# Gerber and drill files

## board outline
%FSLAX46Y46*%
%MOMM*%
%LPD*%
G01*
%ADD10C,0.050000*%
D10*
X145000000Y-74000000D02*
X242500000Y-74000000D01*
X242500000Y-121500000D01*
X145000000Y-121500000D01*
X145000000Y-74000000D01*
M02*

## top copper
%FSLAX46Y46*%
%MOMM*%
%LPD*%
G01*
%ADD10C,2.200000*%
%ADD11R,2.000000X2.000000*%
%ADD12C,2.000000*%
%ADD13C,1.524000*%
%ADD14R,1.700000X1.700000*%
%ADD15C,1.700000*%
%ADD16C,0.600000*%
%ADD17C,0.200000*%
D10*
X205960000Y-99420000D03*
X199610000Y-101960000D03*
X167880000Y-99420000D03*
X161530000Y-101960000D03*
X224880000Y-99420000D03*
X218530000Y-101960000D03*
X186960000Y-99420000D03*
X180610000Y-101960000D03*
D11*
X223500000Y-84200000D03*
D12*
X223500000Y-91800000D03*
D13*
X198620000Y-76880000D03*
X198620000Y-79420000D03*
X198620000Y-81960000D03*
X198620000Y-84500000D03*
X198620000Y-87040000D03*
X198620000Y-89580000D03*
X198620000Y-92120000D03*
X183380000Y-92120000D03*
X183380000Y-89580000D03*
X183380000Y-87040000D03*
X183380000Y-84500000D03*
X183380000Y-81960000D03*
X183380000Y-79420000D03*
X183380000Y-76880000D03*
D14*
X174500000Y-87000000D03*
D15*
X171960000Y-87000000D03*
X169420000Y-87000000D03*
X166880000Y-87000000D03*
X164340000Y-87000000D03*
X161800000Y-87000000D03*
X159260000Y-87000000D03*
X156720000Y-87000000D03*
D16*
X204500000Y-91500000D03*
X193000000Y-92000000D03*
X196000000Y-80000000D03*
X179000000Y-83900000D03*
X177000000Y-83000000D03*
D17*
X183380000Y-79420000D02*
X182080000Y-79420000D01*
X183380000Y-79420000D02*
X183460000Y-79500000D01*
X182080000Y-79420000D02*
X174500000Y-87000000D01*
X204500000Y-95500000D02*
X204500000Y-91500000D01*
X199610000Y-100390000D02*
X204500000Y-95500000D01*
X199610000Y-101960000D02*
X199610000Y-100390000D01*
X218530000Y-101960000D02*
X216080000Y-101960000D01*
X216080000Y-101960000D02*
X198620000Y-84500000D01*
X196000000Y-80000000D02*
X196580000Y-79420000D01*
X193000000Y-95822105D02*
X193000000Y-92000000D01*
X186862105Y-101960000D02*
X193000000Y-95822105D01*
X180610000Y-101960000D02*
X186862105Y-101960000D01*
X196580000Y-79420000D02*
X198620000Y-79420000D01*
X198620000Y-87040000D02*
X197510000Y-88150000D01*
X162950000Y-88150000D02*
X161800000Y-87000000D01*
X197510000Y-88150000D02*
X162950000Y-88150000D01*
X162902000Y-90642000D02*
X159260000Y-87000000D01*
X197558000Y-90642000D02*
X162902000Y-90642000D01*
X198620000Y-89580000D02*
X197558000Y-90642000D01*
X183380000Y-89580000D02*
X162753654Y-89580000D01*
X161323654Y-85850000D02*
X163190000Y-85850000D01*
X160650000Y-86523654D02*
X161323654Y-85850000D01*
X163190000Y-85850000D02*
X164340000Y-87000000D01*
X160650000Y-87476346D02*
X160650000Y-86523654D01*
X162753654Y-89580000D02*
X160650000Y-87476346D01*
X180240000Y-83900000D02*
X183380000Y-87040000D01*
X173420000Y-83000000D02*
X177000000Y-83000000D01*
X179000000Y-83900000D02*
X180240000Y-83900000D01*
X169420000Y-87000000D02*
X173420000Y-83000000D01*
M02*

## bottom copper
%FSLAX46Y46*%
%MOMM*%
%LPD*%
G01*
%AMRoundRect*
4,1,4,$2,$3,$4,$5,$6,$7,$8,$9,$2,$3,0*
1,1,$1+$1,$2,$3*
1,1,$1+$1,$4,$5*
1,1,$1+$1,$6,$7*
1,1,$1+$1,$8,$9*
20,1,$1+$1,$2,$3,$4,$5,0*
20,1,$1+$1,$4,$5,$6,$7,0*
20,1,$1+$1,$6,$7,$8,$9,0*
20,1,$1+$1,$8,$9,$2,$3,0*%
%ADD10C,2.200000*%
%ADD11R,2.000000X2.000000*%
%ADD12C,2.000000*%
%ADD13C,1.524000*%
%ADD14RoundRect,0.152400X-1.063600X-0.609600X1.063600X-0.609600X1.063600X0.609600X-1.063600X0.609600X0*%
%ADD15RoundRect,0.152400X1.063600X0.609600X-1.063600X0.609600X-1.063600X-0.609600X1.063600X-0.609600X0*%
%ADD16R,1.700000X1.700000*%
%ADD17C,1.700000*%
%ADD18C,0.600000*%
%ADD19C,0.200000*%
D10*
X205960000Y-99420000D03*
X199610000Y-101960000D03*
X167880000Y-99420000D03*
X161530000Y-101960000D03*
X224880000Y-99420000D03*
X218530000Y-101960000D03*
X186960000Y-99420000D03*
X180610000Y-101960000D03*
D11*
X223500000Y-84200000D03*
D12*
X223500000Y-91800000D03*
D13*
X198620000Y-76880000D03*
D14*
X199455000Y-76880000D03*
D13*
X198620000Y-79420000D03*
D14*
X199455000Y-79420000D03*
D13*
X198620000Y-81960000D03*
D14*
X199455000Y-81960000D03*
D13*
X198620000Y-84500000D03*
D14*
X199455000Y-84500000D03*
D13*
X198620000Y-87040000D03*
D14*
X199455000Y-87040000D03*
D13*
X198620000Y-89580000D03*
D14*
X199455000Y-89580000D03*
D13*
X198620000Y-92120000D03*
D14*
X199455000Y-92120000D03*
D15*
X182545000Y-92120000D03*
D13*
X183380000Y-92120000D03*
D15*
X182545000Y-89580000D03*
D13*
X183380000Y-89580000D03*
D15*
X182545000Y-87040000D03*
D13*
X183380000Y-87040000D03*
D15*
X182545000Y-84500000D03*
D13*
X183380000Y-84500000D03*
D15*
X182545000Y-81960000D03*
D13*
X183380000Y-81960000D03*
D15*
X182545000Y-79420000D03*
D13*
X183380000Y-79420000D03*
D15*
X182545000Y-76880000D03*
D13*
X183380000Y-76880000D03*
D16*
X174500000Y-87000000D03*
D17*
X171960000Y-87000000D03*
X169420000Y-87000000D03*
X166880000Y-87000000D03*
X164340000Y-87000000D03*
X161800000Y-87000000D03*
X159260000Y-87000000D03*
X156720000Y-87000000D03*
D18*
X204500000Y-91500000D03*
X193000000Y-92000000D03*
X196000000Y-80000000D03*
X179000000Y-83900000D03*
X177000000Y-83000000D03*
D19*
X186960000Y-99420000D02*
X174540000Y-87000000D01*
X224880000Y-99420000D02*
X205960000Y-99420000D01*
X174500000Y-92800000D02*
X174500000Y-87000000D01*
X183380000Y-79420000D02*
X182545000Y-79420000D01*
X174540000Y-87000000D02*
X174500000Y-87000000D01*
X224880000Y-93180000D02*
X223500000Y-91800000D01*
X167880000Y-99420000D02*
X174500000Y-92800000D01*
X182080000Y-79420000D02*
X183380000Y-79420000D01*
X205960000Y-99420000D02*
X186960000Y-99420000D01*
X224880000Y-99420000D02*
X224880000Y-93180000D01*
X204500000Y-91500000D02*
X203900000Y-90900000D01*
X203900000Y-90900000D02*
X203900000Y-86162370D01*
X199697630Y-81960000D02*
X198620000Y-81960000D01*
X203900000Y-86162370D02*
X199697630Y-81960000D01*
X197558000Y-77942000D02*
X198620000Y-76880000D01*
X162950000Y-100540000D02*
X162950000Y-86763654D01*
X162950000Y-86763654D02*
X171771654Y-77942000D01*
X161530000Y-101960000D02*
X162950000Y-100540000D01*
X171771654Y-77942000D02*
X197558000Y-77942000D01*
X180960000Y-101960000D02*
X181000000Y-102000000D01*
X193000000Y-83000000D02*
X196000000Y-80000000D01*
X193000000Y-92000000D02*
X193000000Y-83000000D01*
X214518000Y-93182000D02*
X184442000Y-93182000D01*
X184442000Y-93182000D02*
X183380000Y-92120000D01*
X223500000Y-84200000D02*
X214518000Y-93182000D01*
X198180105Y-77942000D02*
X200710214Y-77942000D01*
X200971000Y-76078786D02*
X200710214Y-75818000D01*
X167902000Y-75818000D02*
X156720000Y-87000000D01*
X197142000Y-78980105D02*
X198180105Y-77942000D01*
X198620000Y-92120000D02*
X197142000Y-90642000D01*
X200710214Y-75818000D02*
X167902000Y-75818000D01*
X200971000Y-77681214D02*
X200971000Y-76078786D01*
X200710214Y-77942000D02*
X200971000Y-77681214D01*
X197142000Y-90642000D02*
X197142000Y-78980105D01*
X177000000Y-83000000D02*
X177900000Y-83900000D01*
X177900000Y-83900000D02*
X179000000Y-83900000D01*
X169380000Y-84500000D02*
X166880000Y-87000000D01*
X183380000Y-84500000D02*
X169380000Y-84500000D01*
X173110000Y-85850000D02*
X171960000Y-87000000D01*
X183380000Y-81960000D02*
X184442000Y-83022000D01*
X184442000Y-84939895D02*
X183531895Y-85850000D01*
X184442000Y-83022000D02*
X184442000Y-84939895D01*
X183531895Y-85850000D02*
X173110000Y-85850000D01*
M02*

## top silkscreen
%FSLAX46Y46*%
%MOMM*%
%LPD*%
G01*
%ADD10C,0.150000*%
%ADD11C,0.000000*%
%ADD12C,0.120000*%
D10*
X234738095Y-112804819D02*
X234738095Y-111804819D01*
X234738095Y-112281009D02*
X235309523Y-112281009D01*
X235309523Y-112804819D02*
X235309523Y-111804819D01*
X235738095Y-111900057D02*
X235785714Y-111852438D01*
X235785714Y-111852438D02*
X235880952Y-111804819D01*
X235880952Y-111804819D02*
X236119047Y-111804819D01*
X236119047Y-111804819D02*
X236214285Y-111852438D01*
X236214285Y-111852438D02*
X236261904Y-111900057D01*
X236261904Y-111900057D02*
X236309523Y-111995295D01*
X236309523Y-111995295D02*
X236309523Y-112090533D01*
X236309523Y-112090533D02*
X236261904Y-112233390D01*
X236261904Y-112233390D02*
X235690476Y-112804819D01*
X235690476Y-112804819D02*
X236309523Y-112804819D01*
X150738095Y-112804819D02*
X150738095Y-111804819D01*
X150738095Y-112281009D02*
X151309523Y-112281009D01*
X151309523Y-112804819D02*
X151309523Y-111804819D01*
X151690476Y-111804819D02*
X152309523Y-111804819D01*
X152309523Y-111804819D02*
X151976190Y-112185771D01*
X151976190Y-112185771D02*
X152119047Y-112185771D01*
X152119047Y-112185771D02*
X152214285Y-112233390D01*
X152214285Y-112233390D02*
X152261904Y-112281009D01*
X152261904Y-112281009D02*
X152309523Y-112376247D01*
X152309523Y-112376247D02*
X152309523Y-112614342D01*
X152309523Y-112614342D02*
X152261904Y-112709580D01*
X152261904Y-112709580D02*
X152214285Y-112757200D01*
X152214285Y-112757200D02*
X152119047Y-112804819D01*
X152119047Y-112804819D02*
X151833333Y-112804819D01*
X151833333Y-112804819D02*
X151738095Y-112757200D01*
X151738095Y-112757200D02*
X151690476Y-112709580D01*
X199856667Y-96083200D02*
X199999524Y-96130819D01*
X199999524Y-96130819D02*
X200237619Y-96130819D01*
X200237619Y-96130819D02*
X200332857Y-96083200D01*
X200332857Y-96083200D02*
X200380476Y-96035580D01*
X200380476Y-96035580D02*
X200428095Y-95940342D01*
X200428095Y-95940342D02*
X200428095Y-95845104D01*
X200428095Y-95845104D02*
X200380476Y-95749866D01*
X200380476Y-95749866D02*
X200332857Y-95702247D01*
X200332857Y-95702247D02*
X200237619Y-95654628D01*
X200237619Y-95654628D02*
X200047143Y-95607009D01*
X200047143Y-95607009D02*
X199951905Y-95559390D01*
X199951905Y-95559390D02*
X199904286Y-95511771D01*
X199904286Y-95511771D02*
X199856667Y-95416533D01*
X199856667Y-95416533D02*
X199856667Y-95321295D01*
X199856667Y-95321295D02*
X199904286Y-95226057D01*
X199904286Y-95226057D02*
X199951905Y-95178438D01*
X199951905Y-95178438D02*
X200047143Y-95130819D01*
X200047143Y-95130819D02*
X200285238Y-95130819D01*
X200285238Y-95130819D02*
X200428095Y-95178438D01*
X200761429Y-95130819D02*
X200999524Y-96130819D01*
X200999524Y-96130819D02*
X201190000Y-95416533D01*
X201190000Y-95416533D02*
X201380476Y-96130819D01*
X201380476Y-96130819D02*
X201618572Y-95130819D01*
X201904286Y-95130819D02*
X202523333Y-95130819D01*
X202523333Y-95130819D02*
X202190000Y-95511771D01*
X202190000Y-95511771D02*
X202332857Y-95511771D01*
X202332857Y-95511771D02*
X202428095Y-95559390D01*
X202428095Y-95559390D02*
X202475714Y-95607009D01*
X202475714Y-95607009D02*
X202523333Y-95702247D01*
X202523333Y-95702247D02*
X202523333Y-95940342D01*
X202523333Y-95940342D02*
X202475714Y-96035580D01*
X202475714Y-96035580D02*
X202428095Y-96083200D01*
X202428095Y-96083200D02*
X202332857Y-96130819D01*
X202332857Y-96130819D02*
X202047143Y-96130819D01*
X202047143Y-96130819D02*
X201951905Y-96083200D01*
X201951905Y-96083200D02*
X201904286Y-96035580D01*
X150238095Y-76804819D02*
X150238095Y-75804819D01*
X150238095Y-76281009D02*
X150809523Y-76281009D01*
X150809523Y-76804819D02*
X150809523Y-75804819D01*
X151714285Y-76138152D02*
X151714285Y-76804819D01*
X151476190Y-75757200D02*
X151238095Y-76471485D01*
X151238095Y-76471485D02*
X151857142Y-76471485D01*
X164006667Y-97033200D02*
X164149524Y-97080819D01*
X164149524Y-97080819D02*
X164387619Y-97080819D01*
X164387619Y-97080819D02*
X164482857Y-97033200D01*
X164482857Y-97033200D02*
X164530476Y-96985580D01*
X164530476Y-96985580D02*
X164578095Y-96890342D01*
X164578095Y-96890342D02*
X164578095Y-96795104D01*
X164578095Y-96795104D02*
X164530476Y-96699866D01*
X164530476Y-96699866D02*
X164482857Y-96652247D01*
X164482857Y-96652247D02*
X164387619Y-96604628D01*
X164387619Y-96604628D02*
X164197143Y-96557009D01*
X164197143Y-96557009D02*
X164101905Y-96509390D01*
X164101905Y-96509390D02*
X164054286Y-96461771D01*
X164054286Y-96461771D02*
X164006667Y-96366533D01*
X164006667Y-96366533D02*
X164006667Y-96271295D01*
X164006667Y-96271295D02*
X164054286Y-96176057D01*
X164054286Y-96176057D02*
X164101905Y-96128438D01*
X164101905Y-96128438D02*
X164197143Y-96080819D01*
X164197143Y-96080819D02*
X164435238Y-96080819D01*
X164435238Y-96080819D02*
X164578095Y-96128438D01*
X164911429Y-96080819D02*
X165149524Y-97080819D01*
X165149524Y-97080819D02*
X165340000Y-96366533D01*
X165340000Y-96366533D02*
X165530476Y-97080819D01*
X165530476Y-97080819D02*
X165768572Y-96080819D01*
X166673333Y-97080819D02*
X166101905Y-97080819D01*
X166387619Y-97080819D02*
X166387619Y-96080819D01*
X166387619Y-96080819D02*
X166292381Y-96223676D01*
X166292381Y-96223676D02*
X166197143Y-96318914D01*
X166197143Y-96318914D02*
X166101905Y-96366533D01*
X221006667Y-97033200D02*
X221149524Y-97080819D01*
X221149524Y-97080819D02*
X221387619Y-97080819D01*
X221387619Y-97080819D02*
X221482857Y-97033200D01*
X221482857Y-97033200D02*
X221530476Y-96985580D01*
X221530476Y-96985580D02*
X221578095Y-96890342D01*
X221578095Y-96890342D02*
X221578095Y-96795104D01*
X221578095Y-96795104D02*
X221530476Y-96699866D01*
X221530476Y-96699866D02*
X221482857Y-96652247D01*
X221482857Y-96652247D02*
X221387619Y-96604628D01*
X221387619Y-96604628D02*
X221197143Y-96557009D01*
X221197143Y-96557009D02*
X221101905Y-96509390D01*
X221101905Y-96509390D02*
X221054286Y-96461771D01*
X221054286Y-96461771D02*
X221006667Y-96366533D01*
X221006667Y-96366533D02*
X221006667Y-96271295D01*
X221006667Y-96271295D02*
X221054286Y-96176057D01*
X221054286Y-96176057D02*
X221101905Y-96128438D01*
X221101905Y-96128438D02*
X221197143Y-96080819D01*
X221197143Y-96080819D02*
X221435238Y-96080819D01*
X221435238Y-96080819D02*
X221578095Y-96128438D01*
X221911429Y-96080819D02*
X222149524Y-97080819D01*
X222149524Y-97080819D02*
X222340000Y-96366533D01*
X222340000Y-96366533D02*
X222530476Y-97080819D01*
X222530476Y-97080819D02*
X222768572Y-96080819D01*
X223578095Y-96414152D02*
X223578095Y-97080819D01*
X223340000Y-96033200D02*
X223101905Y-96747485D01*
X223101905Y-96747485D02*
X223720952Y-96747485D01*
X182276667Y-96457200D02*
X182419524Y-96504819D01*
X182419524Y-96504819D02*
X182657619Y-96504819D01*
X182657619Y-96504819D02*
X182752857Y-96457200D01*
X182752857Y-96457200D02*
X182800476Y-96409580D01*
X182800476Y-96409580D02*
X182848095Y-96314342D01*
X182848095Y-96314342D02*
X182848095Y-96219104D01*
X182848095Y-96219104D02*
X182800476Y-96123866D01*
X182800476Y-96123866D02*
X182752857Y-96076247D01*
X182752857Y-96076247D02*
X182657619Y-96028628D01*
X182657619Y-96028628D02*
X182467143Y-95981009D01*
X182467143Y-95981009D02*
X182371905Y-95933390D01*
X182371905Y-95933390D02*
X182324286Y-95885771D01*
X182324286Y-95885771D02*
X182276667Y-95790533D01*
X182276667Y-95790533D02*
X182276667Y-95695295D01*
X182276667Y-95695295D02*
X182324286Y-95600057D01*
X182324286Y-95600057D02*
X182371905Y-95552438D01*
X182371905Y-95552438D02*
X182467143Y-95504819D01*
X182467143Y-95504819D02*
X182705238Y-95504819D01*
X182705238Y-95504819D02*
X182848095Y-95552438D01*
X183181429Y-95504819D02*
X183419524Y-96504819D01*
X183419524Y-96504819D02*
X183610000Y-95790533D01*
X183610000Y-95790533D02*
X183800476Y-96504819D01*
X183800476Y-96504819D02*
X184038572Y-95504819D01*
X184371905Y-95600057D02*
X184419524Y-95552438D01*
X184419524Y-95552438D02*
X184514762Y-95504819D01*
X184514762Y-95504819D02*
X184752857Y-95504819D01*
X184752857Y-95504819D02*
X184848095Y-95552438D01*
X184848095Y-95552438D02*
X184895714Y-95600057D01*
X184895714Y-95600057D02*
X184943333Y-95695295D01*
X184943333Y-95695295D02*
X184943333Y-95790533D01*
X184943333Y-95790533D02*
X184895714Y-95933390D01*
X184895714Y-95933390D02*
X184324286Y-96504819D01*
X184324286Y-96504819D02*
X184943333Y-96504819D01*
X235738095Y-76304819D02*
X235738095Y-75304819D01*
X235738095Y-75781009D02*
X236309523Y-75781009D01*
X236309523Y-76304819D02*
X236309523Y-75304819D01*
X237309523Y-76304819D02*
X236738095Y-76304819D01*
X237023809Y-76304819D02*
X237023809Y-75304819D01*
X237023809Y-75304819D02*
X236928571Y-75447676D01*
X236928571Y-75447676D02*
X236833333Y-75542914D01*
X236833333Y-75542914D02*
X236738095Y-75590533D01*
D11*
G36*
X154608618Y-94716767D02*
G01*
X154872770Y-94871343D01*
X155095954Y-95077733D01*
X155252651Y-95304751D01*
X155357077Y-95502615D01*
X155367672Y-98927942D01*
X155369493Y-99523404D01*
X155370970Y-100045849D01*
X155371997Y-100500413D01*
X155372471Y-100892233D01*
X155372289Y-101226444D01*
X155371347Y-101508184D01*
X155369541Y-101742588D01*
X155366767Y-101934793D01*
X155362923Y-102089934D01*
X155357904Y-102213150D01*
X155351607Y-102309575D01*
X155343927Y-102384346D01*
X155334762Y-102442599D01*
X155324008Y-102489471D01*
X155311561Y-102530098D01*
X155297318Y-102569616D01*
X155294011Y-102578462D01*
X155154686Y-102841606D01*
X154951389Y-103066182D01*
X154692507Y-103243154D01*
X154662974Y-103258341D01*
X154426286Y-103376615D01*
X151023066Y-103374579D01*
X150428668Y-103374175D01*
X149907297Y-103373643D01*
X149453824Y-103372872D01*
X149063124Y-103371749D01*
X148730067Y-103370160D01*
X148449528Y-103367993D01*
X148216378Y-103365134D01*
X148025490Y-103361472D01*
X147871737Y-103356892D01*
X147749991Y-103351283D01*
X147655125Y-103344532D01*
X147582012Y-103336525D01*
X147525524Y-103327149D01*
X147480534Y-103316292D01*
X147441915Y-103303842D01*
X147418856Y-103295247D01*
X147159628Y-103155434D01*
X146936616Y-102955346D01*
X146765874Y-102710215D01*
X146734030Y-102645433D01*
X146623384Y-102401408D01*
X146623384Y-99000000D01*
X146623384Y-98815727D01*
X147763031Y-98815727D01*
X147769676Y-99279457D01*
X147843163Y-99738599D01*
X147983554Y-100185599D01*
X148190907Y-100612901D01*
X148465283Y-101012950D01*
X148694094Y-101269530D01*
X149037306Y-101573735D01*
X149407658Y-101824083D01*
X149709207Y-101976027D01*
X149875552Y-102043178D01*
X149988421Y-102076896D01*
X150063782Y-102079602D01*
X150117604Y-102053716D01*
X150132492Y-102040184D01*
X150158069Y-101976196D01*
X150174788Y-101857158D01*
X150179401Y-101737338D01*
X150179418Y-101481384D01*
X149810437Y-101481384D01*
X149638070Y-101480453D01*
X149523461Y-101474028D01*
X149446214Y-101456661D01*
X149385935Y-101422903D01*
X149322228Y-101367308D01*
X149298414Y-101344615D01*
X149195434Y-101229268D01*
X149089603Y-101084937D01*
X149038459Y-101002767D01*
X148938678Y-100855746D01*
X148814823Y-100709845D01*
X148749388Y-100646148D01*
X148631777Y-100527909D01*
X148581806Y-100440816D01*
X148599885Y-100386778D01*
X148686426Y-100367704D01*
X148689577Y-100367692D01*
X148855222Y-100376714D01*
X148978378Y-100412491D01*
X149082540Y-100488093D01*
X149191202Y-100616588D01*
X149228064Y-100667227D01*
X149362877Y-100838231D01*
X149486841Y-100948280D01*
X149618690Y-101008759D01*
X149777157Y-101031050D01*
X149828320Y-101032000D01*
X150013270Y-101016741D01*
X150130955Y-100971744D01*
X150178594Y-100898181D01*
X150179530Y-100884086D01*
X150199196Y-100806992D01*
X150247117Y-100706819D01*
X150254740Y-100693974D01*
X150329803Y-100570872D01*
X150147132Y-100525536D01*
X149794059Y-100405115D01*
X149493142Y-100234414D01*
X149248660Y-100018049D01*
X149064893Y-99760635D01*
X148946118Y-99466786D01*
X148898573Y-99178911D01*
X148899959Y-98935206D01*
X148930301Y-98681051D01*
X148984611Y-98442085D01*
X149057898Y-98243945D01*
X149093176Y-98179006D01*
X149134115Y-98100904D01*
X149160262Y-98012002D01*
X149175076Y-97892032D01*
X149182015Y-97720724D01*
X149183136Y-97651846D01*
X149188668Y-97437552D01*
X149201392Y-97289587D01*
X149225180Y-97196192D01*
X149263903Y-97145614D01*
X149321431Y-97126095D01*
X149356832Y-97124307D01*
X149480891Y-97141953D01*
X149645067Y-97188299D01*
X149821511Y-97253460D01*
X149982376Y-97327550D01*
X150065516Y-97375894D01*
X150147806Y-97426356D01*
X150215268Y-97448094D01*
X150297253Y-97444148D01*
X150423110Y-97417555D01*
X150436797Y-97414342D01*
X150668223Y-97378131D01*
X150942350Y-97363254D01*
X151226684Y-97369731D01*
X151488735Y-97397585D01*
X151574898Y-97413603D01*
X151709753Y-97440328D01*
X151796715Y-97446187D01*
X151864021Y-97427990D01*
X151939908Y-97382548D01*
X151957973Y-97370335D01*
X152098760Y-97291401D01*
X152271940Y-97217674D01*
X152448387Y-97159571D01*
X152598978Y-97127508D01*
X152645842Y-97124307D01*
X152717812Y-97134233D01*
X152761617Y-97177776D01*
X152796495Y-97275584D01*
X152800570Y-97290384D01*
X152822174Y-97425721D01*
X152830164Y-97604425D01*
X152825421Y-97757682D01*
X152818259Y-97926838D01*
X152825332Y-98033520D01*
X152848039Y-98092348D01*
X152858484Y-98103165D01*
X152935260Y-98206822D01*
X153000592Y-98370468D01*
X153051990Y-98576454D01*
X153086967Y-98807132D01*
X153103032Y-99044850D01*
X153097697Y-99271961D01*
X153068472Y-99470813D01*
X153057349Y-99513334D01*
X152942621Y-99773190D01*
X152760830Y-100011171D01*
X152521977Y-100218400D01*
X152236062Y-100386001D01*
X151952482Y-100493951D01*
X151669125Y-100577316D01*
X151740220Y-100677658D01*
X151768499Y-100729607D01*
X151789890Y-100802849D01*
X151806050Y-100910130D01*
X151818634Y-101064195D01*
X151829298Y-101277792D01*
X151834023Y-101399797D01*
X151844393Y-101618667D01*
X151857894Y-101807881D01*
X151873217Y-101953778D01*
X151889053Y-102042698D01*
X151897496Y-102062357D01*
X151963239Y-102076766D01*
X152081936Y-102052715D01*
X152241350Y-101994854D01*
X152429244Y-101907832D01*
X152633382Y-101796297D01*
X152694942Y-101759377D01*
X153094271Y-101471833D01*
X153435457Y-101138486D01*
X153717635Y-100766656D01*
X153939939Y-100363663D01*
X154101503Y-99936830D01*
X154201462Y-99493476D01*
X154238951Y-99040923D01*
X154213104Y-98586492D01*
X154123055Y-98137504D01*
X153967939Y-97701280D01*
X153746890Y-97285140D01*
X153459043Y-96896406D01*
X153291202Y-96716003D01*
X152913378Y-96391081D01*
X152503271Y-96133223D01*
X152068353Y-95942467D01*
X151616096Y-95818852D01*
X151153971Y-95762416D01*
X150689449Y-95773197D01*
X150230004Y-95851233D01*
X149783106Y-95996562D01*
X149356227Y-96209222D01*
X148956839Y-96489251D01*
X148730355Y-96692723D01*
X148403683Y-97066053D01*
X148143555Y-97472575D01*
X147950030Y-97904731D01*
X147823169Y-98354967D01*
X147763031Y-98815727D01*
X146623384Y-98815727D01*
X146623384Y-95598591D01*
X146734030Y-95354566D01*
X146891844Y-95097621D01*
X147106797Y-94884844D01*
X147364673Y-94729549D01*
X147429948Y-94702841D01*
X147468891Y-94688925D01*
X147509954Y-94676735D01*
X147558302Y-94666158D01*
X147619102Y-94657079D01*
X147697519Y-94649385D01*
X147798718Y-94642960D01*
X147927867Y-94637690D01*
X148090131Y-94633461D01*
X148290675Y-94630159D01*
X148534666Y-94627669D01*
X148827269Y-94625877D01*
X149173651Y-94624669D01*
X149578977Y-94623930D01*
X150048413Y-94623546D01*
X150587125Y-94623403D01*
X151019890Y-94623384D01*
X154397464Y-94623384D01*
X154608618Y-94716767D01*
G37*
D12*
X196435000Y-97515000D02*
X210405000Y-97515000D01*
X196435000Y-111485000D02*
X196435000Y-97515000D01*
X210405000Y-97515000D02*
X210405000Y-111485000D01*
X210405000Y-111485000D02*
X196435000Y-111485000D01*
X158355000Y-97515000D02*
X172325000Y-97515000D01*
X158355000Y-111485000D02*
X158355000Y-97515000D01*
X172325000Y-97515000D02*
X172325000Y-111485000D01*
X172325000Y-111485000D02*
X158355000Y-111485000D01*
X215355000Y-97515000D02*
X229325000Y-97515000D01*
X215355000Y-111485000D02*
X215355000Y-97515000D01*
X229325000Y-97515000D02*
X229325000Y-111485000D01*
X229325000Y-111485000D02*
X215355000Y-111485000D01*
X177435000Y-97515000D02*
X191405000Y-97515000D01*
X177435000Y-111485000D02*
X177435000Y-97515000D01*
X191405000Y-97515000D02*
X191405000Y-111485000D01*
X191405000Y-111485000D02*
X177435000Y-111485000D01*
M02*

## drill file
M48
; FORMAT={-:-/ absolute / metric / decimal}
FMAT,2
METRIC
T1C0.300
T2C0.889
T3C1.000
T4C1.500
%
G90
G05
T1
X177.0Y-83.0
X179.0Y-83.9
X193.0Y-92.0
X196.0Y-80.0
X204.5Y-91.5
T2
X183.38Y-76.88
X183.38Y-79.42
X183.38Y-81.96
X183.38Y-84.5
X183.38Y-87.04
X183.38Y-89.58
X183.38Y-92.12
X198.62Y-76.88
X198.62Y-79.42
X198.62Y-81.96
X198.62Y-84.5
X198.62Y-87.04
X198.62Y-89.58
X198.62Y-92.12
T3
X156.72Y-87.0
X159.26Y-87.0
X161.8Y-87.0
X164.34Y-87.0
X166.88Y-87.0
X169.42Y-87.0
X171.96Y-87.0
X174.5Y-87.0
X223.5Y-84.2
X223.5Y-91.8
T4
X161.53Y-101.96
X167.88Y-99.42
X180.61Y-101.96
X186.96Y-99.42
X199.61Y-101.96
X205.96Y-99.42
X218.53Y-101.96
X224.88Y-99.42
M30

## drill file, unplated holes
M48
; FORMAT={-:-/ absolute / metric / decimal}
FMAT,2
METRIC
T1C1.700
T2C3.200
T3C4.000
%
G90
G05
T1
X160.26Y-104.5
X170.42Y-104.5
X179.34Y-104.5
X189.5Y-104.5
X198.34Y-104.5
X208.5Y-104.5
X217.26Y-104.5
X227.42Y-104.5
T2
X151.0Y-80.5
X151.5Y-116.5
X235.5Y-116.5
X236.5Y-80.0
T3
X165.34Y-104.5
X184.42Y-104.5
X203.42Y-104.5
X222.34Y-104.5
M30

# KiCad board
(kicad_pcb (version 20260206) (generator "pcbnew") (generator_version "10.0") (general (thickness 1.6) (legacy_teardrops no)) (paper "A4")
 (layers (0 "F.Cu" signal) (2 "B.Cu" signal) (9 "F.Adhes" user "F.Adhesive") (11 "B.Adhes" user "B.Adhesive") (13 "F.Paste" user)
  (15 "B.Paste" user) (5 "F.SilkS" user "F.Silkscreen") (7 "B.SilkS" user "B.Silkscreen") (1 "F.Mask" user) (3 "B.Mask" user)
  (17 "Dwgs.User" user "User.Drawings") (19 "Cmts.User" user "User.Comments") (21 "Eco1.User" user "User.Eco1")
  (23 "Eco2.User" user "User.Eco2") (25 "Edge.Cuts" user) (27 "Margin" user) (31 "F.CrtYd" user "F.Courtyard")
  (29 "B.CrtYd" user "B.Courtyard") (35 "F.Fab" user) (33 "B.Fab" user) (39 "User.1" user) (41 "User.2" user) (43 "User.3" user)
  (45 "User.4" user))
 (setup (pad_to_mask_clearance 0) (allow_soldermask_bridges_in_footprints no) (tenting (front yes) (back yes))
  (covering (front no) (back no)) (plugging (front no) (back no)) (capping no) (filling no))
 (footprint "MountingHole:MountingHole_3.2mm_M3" (layer "F.Cu") (at 235.5 116.5)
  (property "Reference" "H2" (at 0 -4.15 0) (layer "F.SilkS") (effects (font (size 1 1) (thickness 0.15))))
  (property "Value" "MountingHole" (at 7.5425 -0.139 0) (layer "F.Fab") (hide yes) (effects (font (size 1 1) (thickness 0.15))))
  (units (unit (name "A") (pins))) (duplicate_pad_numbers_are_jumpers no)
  (pad "" np_thru_hole circle (at 0 0) (size 3.2 3.2) (drill 3.2) (layers "*.Cu" "*.Mask")))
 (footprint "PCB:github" (layer "F.Cu") (at 151 99)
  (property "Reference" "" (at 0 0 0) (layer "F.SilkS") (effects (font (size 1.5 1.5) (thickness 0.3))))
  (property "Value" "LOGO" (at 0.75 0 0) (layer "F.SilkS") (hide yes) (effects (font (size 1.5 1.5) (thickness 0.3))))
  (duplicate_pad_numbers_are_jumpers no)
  (fp_poly
   (pts (xy 3.608618 -4.283233) (xy 3.87277 -4.128657) (xy 4.095954 -3.922267) (xy 4.252651 -3.695249) (xy 4.357077 -3.497385)
    (xy 4.367672 -0.072058) (xy 4.369493 0.523404) (xy 4.37097 1.045849) (xy 4.371997 1.500413) (xy 4.372471 1.892233)
    (xy 4.372289 2.226444) (xy 4.371347 2.508184) (xy 4.369541 2.742588) (xy 4.366767 2.934793) (xy 4.362923 3.089934) (xy 4.357904 3.21315)
    (xy 4.351607 3.309575) (xy 4.343927 3.384346) (xy 4.334762 3.442599) (xy 4.324008 3.489471) (xy 4.311561 3.530098)
    (xy 4.297318 3.569616) (xy 4.294011 3.578462) (xy 4.154686 3.841606) (xy 3.951389 4.066182) (xy 3.692507 4.243154)
    (xy 3.662974 4.258341) (xy 3.426286 4.376615) (xy 0.023066 4.374579) (xy -0.571332 4.374175) (xy -1.092703 4.373643)
    (xy -1.546176 4.372872) (xy -1.936876 4.371749) (xy -2.269933 4.37016) (xy -2.550472 4.367993) (xy -2.783622 4.365134)
    (xy -2.97451 4.361472) (xy -3.128263 4.356892) (xy -3.250009 4.351283) (xy -3.344875 4.344532) (xy -3.417988 4.336525)
    (xy -3.474476 4.327149) (xy -3.519466 4.316292) (xy -3.558085 4.303842) (xy -3.581144 4.295247) (xy -3.840372 4.155434)
    (xy -4.063384 3.955346) (xy -4.234126 3.710215) (xy -4.26597 3.645433) (xy -4.376616 3.401408) (xy -4.376616 0) (xy -4.376616 -0.184273)
    (xy -3.236969 -0.184273) (xy -3.230324 0.279457) (xy -3.156837 0.738599) (xy -3.016446 1.185599) (xy -2.809093 1.612901)
    (xy -2.534717 2.01295) (xy -2.305906 2.26953) (xy -1.962694 2.573735) (xy -1.592342 2.824083) (xy -1.290793 2.976027)
    (xy -1.124448 3.043178) (xy -1.011579 3.076896) (xy -0.936218 3.079602) (xy -0.882396 3.053716) (xy -0.867508 3.040184)
    (xy -0.841931 2.976196) (xy -0.825212 2.857158) (xy -0.820599 2.737338) (xy -0.820582 2.481384) (xy -1.189563 2.481384)
    (xy -1.36193 2.480453) (xy -1.476539 2.474028) (xy -1.553786 2.456661) (xy -1.614065 2.422903) (xy -1.677772 2.367308)
    (xy -1.701586 2.344615) (xy -1.804566 2.229268) (xy -1.910397 2.084937) (xy -1.961541 2.002767) (xy -2.061322 1.855746)
    (xy -2.185177 1.709845) (xy -2.250612 1.646148) (xy -2.368223 1.527909) (xy -2.418194 1.440816) (xy -2.400115 1.386778)
    (xy -2.313574 1.367704) (xy -2.310423 1.367692) (xy -2.144778 1.376714) (xy -2.021622 1.412491) (xy -1.91746 1.488093)
    (xy -1.808798 1.616588) (xy -1.771936 1.667227) (xy -1.637123 1.838231) (xy -1.513159 1.94828) (xy -1.38131 2.008759)
    (xy -1.222843 2.03105) (xy -1.17168 2.032) (xy -0.98673 2.016741) (xy -0.869045 1.971744) (xy -0.821406 1.898181) (xy -0.82047 1.884086)
    (xy -0.800804 1.806992) (xy -0.752883 1.706819) (xy -0.74526 1.693974) (xy -0.670197 1.570872) (xy -0.852868 1.525536)
    (xy -1.205941 1.405115) (xy -1.506858 1.234414) (xy -1.75134 1.018049) (xy -1.935107 0.760635) (xy -2.053882 0.466786)
    (xy -2.101427 0.178911) (xy -2.100041 -0.064794) (xy -2.069699 -0.318949) (xy -2.015389 -0.557915) (xy -1.942102 -0.756055)
    (xy -1.906824 -0.820994) (xy -1.865885 -0.899096) (xy -1.839738 -0.987998) (xy -1.824924 -1.107968) (xy -1.817985 -1.279276)
    (xy -1.816864 -1.348154) (xy -1.811332 -1.562448) (xy -1.798608 -1.710413) (xy -1.77482 -1.803808) (xy -1.736097 -1.854386)
    (xy -1.678569 -1.873905) (xy -1.643168 -1.875693) (xy -1.519109 -1.858047) (xy -1.354933 -1.811701) (xy -1.178489 -1.74654)
    (xy -1.017624 -1.67245) (xy -0.934484 -1.624106) (xy -0.852194 -1.573644) (xy -0.784732 -1.551906) (xy -0.702747 -1.555852)
    (xy -0.57689 -1.582445) (xy -0.563203 -1.585658) (xy -0.331777 -1.621869) (xy -0.05765 -1.636746) (xy 0.226684 -1.630269)
    (xy 0.488735 -1.602415) (xy 0.574898 -1.586397) (xy 0.709753 -1.559672) (xy 0.796715 -1.553813) (xy 0.864021 -1.57201)
    (xy 0.939908 -1.617452) (xy 0.957973 -1.629665) (xy 1.09876 -1.708599) (xy 1.27194 -1.782326) (xy 1.448387 -1.840429)
    (xy 1.598978 -1.872492) (xy 1.645842 -1.875693) (xy 1.717812 -1.865767) (xy 1.761617 -1.822224) (xy 1.796495 -1.724416)
    (xy 1.80057 -1.709616) (xy 1.822174 -1.574279) (xy 1.830164 -1.395575) (xy 1.825421 -1.242318) (xy 1.818259 -1.073162)
    (xy 1.825332 -0.96648) (xy 1.848039 -0.907652) (xy 1.858484 -0.896835) (xy 1.93526 -0.793178) (xy 2.000592 -0.629532)
    (xy 2.05199 -0.423546) (xy 2.086967 -0.192868) (xy 2.103032 0.04485) (xy 2.097697 0.271961) (xy 2.068472 0.470813)
    (xy 2.057349 0.513334) (xy 1.942621 0.77319) (xy 1.76083 1.011171) (xy 1.521977 1.2184) (xy 1.236062 1.386001) (xy 0.952482 1.493951)
    (xy 0.669125 1.577316) (xy 0.74022 1.677658) (xy 0.768499 1.729607) (xy 0.78989 1.802849) (xy 0.80605 1.91013) (xy 0.818634 2.064195)
    (xy 0.829298 2.277792) (xy 0.834023 2.399797) (xy 0.844393 2.618667) (xy 0.857894 2.807881) (xy 0.873217 2.953778)
    (xy 0.889053 3.042698) (xy 0.897496 3.062357) (xy 0.963239 3.076766) (xy 1.081936 3.052715) (xy 1.24135 2.994854) (xy 1.429244 2.907832)
    (xy 1.633382 2.796297) (xy 1.694942 2.759377) (xy 2.094271 2.471833) (xy 2.435457 2.138486) (xy 2.717635 1.766656)
    (xy 2.939939 1.363663) (xy 3.101503 0.93683) (xy 3.201462 0.493476) (xy 3.238951 0.040923) (xy 3.213104 -0.413508)
    (xy 3.123055 -0.862496) (xy 2.967939 -1.29872) (xy 2.74689 -1.71486) (xy 2.459043 -2.103594) (xy 2.291202 -2.283997)
    (xy 1.913378 -2.608919) (xy 1.503271 -2.866777) (xy 1.068353 -3.057533) (xy 0.616096 -3.181148) (xy 0.153971 -3.237584)
    (xy -0.310551 -3.226803) (xy -0.769996 -3.148767) (xy -1.216894 -3.003438) (xy -1.643773 -2.790778) (xy -2.043161 -2.510749)
    (xy -2.269645 -2.307277) (xy -2.596317 -1.933947) (xy -2.856445 -1.527425) (xy -3.04997 -1.095269) (xy -3.176831 -0.645033)
    (xy -3.236969 -0.184273) (xy -4.376616 -0.184273) (xy -4.376616 -3.401409) (xy -4.26597 -3.645434) (xy -4.108156 -3.902379)
    (xy -3.893203 -4.115156) (xy -3.635327 -4.270451) (xy -3.570052 -4.297159) (xy -3.531109 -4.311075) (xy -3.490046 -4.323265)
    (xy -3.441698 -4.333842) (xy -3.380898 -4.342921) (xy -3.302481 -4.350615) (xy -3.201282 -4.35704) (xy -3.072133 -4.36231)
    (xy -2.909869 -4.366539) (xy -2.709325 -4.369841) (xy -2.465334 -4.372331) (xy -2.172731 -4.374123) (xy -1.826349 -4.375331)
    (xy -1.421023 -4.37607) (xy -0.951587 -4.376454) (xy -0.412875 -4.376597) (xy 0.01989 -4.376616) (xy 3.397464 -4.376616))
   (stroke (width 0) (type solid)) (fill yes) (layer "F.SilkS")))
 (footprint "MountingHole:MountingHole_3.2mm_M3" (layer "F.Cu") (at 151.5 116.5)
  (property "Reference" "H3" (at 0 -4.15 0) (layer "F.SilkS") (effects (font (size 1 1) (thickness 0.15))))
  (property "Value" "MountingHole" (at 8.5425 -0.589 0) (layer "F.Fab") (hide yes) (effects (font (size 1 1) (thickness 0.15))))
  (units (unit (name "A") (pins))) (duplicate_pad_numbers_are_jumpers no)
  (pad "" np_thru_hole circle (at 0 0) (size 3.2 3.2) (drill 3.2) (layers "*.Cu" "*.Mask")))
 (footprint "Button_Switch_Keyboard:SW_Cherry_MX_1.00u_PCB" (layer "F.Cu") (at 205.96 99.42)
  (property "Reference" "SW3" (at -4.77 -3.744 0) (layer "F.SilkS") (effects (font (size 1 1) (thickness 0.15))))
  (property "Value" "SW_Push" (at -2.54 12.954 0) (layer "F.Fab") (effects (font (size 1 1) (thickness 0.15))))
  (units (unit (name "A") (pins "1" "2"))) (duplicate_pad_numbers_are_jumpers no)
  (fp_line (start -9.525 -1.905) (end 4.445 -1.905) (stroke (width 0.12) (type solid)) (layer "F.SilkS"))
  (fp_line (start -9.525 12.065) (end -9.525 -1.905) (stroke (width 0.12) (type solid)) (layer "F.SilkS"))
  (fp_line (start 4.445 -1.905) (end 4.445 12.065) (stroke (width 0.12) (type solid)) (layer "F.SilkS"))
  (fp_line (start 4.445 12.065) (end -9.525 12.065) (stroke (width 0.12) (type solid)) (layer "F.SilkS"))
  (pad "" np_thru_hole circle (at -7.62 5.08) (size 1.7 1.7) (drill 1.7) (layers "*.Cu" "*.Mask"))
  (pad "" np_thru_hole circle (at -2.54 5.08) (size 4 4) (drill 4) (layers "*.Cu" "*.Mask"))
  (pad "" np_thru_hole circle (at 2.54 5.08) (size 1.7 1.7) (drill 1.7) (layers "*.Cu" "*.Mask"))
  (pad "1" thru_hole circle (at 0 0) (size 2.2 2.2) (drill 1.5) (layers "*.Cu" "*.Mask") (remove_unused_layers no) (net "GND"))
  (pad "2" thru_hole circle (at -6.35 2.54) (size 2.2 2.2) (drill 1.5) (layers "*.Cu" "*.Mask") (remove_unused_layers no)
   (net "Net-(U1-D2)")))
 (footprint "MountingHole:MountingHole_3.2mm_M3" (layer "F.Cu") (at 151 80.5)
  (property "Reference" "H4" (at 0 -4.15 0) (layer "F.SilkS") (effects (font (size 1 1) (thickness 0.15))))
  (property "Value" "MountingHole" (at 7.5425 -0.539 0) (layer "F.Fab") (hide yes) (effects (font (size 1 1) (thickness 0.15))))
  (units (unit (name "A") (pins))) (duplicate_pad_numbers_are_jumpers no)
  (pad "" np_thru_hole circle (at 0 0) (size 3.2 3.2) (drill 3.2) (layers "*.Cu" "*.Mask")))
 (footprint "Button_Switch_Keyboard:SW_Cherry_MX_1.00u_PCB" (layer "F.Cu") (at 167.88 99.42)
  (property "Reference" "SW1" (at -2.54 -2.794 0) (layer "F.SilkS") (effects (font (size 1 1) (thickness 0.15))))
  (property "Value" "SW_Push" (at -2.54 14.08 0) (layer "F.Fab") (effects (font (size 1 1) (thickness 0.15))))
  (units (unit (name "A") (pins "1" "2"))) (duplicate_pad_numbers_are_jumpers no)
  (fp_line (start -9.525 -1.905) (end 4.445 -1.905) (stroke (width 0.12) (type solid)) (layer "F.SilkS"))
  (fp_line (start -9.525 12.065) (end -9.525 -1.905) (stroke (width 0.12) (type solid)) (layer "F.SilkS"))
  (fp_line (start 4.445 -1.905) (end 4.445 12.065) (stroke (width 0.12) (type solid)) (layer "F.SilkS"))
  (fp_line (start 4.445 12.065) (end -9.525 12.065) (stroke (width 0.12) (type solid)) (layer "F.SilkS"))
  (pad "" np_thru_hole circle (at -7.62 5.08) (size 1.7 1.7) (drill 1.7) (layers "*.Cu" "*.Mask"))
  (pad "" np_thru_hole circle (at -2.54 5.08) (size 4 4) (drill 4) (layers "*.Cu" "*.Mask"))
  (pad "" np_thru_hole circle (at 2.54 5.08) (size 1.7 1.7) (drill 1.7) (layers "*.Cu" "*.Mask"))
  (pad "1" thru_hole circle (at 0 0) (size 2.2 2.2) (drill 1.5) (layers "*.Cu" "*.Mask") (remove_unused_layers no) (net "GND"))
  (pad "2" thru_hole circle (at -6.35 2.54) (size 2.2 2.2) (drill 1.5) (layers "*.Cu" "*.Mask") (remove_unused_layers no)
   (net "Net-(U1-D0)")))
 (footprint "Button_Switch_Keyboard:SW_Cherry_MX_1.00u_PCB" (layer "F.Cu") (at 224.88 99.42)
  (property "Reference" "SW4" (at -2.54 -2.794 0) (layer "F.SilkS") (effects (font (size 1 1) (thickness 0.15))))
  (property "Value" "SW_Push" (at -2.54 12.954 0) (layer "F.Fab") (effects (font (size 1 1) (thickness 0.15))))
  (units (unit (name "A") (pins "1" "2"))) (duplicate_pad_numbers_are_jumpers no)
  (fp_line (start -9.525 -1.905) (end 4.445 -1.905) (stroke (width 0.12) (type solid)) (layer "F.SilkS"))
  (fp_line (start -9.525 12.065) (end -9.525 -1.905) (stroke (width 0.12) (type solid)) (layer "F.SilkS"))
  (fp_line (start 4.445 -1.905) (end 4.445 12.065) (stroke (width 0.12) (type solid)) (layer "F.SilkS"))
  (fp_line (start 4.445 12.065) (end -9.525 12.065) (stroke (width 0.12) (type solid)) (layer "F.SilkS"))
  (pad "" np_thru_hole circle (at -7.62 5.08) (size 1.7 1.7) (drill 1.7) (layers "*.Cu" "*.Mask"))
  (pad "" np_thru_hole circle (at -2.54 5.08) (size 4 4) (drill 4) (layers "*.Cu" "*.Mask"))
  (pad "" np_thru_hole circle (at 2.54 5.08) (size 1.7 1.7) (drill 1.7) (layers "*.Cu" "*.Mask"))
  (pad "1" thru_hole circle (at 0 0) (size 2.2 2.2) (drill 1.5) (layers "*.Cu" "*.Mask") (remove_unused_layers no) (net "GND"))
  (pad "2" thru_hole circle (at -6.35 2.54) (size 2.2 2.2) (drill 1.5) (layers "*.Cu" "*.Mask") (remove_unused_layers no)
   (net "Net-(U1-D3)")))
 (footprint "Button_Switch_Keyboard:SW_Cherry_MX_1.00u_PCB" (layer "F.Cu") (at 186.96 99.42)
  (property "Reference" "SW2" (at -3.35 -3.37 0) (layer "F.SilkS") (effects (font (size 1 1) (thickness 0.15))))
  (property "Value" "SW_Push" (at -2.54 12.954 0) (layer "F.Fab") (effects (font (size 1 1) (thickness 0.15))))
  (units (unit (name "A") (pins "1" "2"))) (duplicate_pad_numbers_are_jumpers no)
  (fp_line (start -9.525 -1.905) (end 4.445 -1.905) (stroke (width 0.12) (type solid)) (layer "F.SilkS"))
  (fp_line (start -9.525 12.065) (end -9.525 -1.905) (stroke (width 0.12) (type solid)) (layer "F.SilkS"))
  (fp_line (start 4.445 -1.905) (end 4.445 12.065) (stroke (width 0.12) (type solid)) (layer "F.SilkS"))
  (fp_line (start 4.445 12.065) (end -9.525 12.065) (stroke (width 0.12) (type solid)) (layer "F.SilkS"))
  (pad "" np_thru_hole circle (at -7.62 5.08) (size 1.7 1.7) (drill 1.7) (layers "*.Cu" "*.Mask"))
  (pad "" np_thru_hole circle (at -2.54 5.08) (size 4 4) (drill 4) (layers "*.Cu" "*.Mask"))
  (pad "" np_thru_hole circle (at 2.54 5.08) (size 1.7 1.7) (drill 1.7) (layers "*.Cu" "*.Mask"))
  (pad "1" thru_hole circle (at 0 0) (size 2.2 2.2) (drill 1.5) (layers "*.Cu" "*.Mask") (remove_unused_layers no) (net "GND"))
  (pad "2" thru_hole circle (at -6.35 2.54) (size 2.2 2.2) (drill 1.5) (layers "*.Cu" "*.Mask") (remove_unused_layers no)
   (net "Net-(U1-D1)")))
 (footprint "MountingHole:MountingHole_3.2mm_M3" (layer "F.Cu") (at 236.5 80)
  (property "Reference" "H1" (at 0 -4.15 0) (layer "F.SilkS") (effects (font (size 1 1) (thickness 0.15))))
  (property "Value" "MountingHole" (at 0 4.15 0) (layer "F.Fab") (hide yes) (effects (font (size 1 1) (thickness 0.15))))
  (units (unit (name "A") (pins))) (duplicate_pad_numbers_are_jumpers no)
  (pad "" np_thru_hole circle (at 0 0) (size 3.2 3.2) (drill 3.2) (layers "*.Cu" "*.Mask")))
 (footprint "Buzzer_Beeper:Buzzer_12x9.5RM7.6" (layer "B.Cu") (at 223.5 84.2 -90)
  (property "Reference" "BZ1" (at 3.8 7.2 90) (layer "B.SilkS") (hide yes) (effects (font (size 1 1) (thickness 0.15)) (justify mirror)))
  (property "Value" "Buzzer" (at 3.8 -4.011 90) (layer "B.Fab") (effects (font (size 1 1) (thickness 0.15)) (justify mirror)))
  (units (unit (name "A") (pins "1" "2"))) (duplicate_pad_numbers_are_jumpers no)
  (pad "1" thru_hole rect (at 0 0 270) (size 2 2) (drill 1) (layers "*.Cu" "*.Mask") (remove_unused_layers no) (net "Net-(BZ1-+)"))
  (pad "2" thru_hole circle (at 7.6 0 270) (size 2 2) (drill 1) (layers "*.Cu" "*.Mask") (remove_unused_layers no) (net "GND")))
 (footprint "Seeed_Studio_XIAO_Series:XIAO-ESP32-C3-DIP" (layer "B.Cu") (at 191 84.5 90)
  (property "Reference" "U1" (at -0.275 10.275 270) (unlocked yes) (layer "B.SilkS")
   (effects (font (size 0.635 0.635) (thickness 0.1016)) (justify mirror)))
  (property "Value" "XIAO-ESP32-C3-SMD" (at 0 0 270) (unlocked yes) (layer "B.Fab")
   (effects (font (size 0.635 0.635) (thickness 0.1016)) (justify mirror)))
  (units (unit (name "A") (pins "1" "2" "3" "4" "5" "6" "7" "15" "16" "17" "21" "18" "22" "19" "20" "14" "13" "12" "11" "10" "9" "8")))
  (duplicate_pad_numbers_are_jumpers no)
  (pad "1" thru_hole circle (at 7.62 7.62) (size 1.524 1.524) (drill 0.889) (layers "*.Cu" "*.Mask") (remove_unused_layers no)
   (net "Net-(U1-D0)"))
  (pad "1" smd roundrect (at 7.62 8.455) (size 2.432 1.524) (layers "B.Cu" "B.Mask") (roundrect_rratio 0.1) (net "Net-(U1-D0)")
   (thermal_bridge_angle 45))
  (pad "2" thru_hole circle (at 5.08 7.62) (size 1.524 1.524) (drill 0.889) (layers "*.Cu" "*.Mask") (remove_unused_layers no)
   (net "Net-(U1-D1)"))
  (pad "2" smd roundrect (at 5.08 8.455) (size 2.432 1.524) (layers "B.Cu" "B.Mask") (roundrect_rratio 0.1) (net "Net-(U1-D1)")
   (thermal_bridge_angle 45))
  (pad "3" thru_hole circle (at 2.54 7.62) (size 1.524 1.524) (drill 0.889) (layers "*.Cu" "*.Mask") (remove_unused_layers no)
   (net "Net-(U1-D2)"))
  (pad "3" smd roundrect (at 2.54 8.455) (size 2.432 1.524) (layers "B.Cu" "B.Mask") (roundrect_rratio 0.1) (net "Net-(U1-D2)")
   (thermal_bridge_angle 45))
  (pad "4" thru_hole circle (at 0 7.62) (size 1.524 1.524) (drill 0.889) (layers "*.Cu" "*.Mask") (remove_unused_layers no)
   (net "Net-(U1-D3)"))
  (pad "4" smd roundrect (at 0 8.455) (size 2.432 1.524) (layers "B.Cu" "B.Mask") (roundrect_rratio 0.1) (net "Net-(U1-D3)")
   (thermal_bridge_angle 45))
  (pad "5" thru_hole circle (at -2.54 7.62) (size 1.524 1.524) (drill 0.889) (layers "*.Cu" "*.Mask") (remove_unused_layers no) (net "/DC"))
  (pad "5" smd roundrect (at -2.54 8.455) (size 2.432 1.524) (layers "B.Cu" "B.Mask") (roundrect_rratio 0.1) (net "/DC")
   (thermal_bridge_angle 45))
  (pad "6" thru_hole circle (at -5.08 7.62) (size 1.524 1.524) (drill 0.889) (layers "*.Cu" "*.Mask") (remove_unused_layers no) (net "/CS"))
  (pad "6" smd roundrect (at -5.08 8.455) (size 2.432 1.524) (layers "B.Cu" "B.Mask") (roundrect_rratio 0.1) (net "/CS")
   (thermal_bridge_angle 45))
  (pad "7" thru_hole circle (at -7.62 7.62) (size 1.524 1.524) (drill 0.889) (layers "*.Cu" "*.Mask") (remove_unused_layers no) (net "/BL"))
  (pad "7" smd roundrect (at -7.62 8.455) (size 2.432 1.524) (layers "B.Cu" "B.Mask") (roundrect_rratio 0.1) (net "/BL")
   (thermal_bridge_angle 45))
  (pad "8" smd roundrect (at -7.62 -8.455 180) (size 2.432 1.524) (layers "B.Cu" "B.Mask") (roundrect_rratio 0.1) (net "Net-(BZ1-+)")
   (thermal_bridge_angle 45))
  (pad "8" thru_hole circle (at -7.62 -7.62 180) (size 1.524 1.524) (drill 0.889) (layers "*.Cu" "*.Mask") (remove_unused_layers no)
   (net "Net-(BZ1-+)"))
  (pad "9" smd roundrect (at -5.08 -8.455 180) (size 2.432 1.524) (layers "B.Cu" "B.Mask") (roundrect_rratio 0.1) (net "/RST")
   (thermal_bridge_angle 45))
  (pad "9" thru_hole circle (at -5.08 -7.62 180) (size 1.524 1.524) (drill 0.889) (layers "*.Cu" "*.Mask") (remove_unused_layers no)
   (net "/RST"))
  (pad "10" smd roundrect (at -2.54 -8.455 180) (size 2.432 1.524) (layers "B.Cu" "B.Mask") (roundrect_rratio 0.1) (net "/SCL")
   (thermal_bridge_angle 45))
  (pad "10" thru_hole circle (at -2.54 -7.62 180) (size 1.524 1.524) (drill 0.889) (layers "*.Cu" "*.Mask") (remove_unused_layers no)
   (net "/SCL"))
  (pad "11" smd roundrect (at 0 -8.455 180) (size 2.432 1.524) (layers "B.Cu" "B.Mask") (roundrect_rratio 0.1) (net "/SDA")
   (thermal_bridge_angle 45))
  (pad "11" thru_hole circle (at 0 -7.62 180) (size 1.524 1.524) (drill 0.889) (layers "*.Cu" "*.Mask") (remove_unused_layers no)
   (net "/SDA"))
  (pad "12" smd roundrect (at 2.54 -8.455 180) (size 2.432 1.524) (layers "B.Cu" "B.Mask") (roundrect_rratio 0.1) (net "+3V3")
   (thermal_bridge_angle 45))
  (pad "12" thru_hole circle (at 2.54 -7.62 180) (size 1.524 1.524) (drill 0.889) (layers "*.Cu" "*.Mask") (remove_unused_layers no)
   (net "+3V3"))
  (pad "13" smd roundrect (at 5.08 -8.455 180) (size 2.432 1.524) (layers "B.Cu" "B.Mask") (roundrect_rratio 0.1) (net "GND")
   (thermal_bridge_angle 45))
  (pad "13" thru_hole circle (at 5.08 -7.62 180) (size 1.524 1.524) (drill 0.889) (layers "*.Cu" "*.Mask") (remove_unused_layers no)
   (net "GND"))
  (pad "14" smd roundrect (at 7.62 -8.455 180) (size 2.432 1.524) (layers "B.Cu" "B.Mask") (roundrect_rratio 0.1)
   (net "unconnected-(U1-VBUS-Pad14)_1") (thermal_bridge_angle 45))
  (pad "14" thru_hole circle (at 7.62 -7.62 180) (size 1.524 1.524) (drill 0.889) (layers "*.Cu" "*.Mask") (remove_unused_layers no)
   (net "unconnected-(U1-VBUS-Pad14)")))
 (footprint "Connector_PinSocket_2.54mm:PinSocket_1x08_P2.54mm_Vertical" (layer "B.Cu") (at 174.5 87 90)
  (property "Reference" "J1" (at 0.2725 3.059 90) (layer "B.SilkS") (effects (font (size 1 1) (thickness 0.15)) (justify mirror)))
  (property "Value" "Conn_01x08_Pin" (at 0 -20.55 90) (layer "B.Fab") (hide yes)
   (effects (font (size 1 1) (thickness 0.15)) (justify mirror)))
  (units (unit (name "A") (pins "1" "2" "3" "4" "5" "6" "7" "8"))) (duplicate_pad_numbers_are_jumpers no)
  (pad "1" thru_hole rect (at 0 0 90) (size 1.7 1.7) (drill 1) (layers "*.Cu" "*.Mask") (remove_unused_layers no) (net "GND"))
  (pad "2" thru_hole circle (at 0 -2.54 90) (size 1.7 1.7) (drill 1) (layers "*.Cu" "*.Mask") (remove_unused_layers no) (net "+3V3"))
  (pad "3" thru_hole circle (at 0 -5.08 90) (size 1.7 1.7) (drill 1) (layers "*.Cu" "*.Mask") (remove_unused_layers no) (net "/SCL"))
  (pad "4" thru_hole circle (at 0 -7.62 90) (size 1.7 1.7) (drill 1) (layers "*.Cu" "*.Mask") (remove_unused_layers no) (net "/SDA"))
  (pad "5" thru_hole circle (at 0 -10.16 90) (size 1.7 1.7) (drill 1) (layers "*.Cu" "*.Mask") (remove_unused_layers no) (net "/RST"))
  (pad "6" thru_hole circle (at 0 -12.7 90) (size 1.7 1.7) (drill 1) (layers "*.Cu" "*.Mask") (remove_unused_layers no) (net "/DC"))
  (pad "7" thru_hole circle (at 0 -15.24 90) (size 1.7 1.7) (drill 1) (layers "*.Cu" "*.Mask") (remove_unused_layers no) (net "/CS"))
  (pad "8" thru_hole circle (at 0 -17.78 90) (size 1.7 1.7) (drill 1) (layers "*.Cu" "*.Mask") (remove_unused_layers no) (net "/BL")))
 (gr_rect (start 145 74) (end 242.5 121.5) (stroke (width 0.05) (type default)) (fill no) (layer "Edge.Cuts"))
 (segment (start 183.38 79.42) (end 182.08 79.42) (width 0.2) (layer "F.Cu") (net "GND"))
 (segment (start 183.38 79.42) (end 183.46 79.5) (width 0.2) (layer "F.Cu") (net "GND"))
 (segment (start 182.08 79.42) (end 174.5 87) (width 0.2) (layer "F.Cu") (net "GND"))
 (segment (start 186.96 99.42) (end 174.54 87) (width 0.2) (layer "B.Cu") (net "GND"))
 (segment (start 224.88 99.42) (end 205.96 99.42) (width 0.2) (layer "B.Cu") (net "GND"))
 (segment (start 174.5 92.8) (end 174.5 87) (width 0.2) (layer "B.Cu") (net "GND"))
 (segment (start 183.38 79.42) (end 182.545 79.42) (width 0.2) (layer "B.Cu") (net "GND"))
 (segment (start 174.54 87) (end 174.5 87) (width 0.2) (layer "B.Cu") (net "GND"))
 (segment (start 224.88 93.18) (end 223.5 91.8) (width 0.2) (layer "B.Cu") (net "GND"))
 (segment (start 167.88 99.42) (end 174.5 92.8) (width 0.2) (layer "B.Cu") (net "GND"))
 (segment (start 182.08 79.42) (end 183.38 79.42) (width 0.2) (layer "B.Cu") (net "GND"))
 (segment (start 205.96 99.42) (end 186.96 99.42) (width 0.2) (layer "B.Cu") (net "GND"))
 (segment (start 224.88 99.42) (end 224.88 93.18) (width 0.2) (layer "B.Cu") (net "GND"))
 (segment (start 204.5 95.5) (end 204.5 91.5) (width 0.2) (layer "F.Cu") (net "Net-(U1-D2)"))
 (segment (start 199.61 100.39) (end 204.5 95.5) (width 0.2) (layer "F.Cu") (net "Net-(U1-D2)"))
 (segment (start 199.61 101.96) (end 199.61 100.39) (width 0.2) (layer "F.Cu") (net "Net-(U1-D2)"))
 (via (at 204.5 91.5) (size 0.6) (drill 0.3) (layers "F.Cu" "B.Cu") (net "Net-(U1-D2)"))
 (segment (start 204.5 91.5) (end 203.9 90.9) (width 0.2) (layer "B.Cu") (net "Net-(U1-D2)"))
 (segment (start 203.9 90.9) (end 203.9 86.16237) (width 0.2) (layer "B.Cu") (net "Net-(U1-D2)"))
 (segment (start 199.69763 81.96) (end 198.62 81.96) (width 0.2) (layer "B.Cu") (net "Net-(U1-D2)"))
 (segment (start 203.9 86.16237) (end 199.69763 81.96) (width 0.2) (layer "B.Cu") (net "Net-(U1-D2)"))
 (segment (start 197.558 77.942) (end 198.62 76.88) (width 0.2) (layer "B.Cu") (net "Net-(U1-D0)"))
 (segment (start 162.95 100.54) (end 162.95 86.763654) (width 0.2) (layer "B.Cu") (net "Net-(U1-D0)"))
 (segment (start 162.95 86.763654) (end 171.771654 77.942) (width 0.2) (layer "B.Cu") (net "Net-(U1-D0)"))
 (segment (start 161.53 101.96) (end 162.95 100.54) (width 0.2) (layer "B.Cu") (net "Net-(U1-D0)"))
 (segment (start 171.771654 77.942) (end 197.558 77.942) (width 0.2) (layer "B.Cu") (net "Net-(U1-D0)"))
 (segment (start 218.53 101.96) (end 216.08 101.96) (width 0.2) (layer "F.Cu") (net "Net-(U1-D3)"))
 (segment (start 216.08 101.96) (end 198.62 84.5) (width 0.2) (layer "F.Cu") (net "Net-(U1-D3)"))
 (segment (start 196 80) (end 196.58 79.42) (width 0.2) (layer "F.Cu") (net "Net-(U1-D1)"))
 (segment (start 193 95.822105) (end 193 92) (width 0.2) (layer "F.Cu") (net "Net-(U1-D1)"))
 (segment (start 186.862105 101.96) (end 193 95.822105) (width 0.2) (layer "F.Cu") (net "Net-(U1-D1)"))
 (segment (start 180.61 101.96) (end 186.862105 101.96) (width 0.2) (layer "F.Cu") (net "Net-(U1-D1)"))
 (segment (start 196.58 79.42) (end 198.62 79.42) (width 0.2) (layer "F.Cu") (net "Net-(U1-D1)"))
 (via (at 193 92) (size 0.6) (drill 0.3) (layers "F.Cu" "B.Cu") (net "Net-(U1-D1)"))
 (via (at 196 80) (size 0.6) (drill 0.3) (layers "F.Cu" "B.Cu") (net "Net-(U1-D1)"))
 (segment (start 180.96 101.96) (end 181 102) (width 0.2) (layer "B.Cu") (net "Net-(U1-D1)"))
 (segment (start 193 83) (end 196 80) (width 0.2) (layer "B.Cu") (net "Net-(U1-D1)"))
 (segment (start 193 92) (end 193 83) (width 0.2) (layer "B.Cu") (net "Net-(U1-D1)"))
 (segment (start 214.518 93.182) (end 184.442 93.182) (width 0.2) (layer "B.Cu") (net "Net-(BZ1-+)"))
 (segment (start 184.442 93.182) (end 183.38 92.12) (width 0.2) (layer "B.Cu") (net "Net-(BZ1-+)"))
 (segment (start 223.5 84.2) (end 214.518 93.182) (width 0.2) (layer "B.Cu") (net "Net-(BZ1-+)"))
 (segment (start 198.62 87.04) (end 197.51 88.15) (width 0.2) (layer "F.Cu") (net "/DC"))
 (segment (start 162.95 88.15) (end 161.8 87) (width 0.2) (layer "F.Cu") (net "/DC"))
 (segment (start 197.51 88.15) (end 162.95 88.15) (width 0.2) (layer "F.Cu") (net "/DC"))
 (segment (start 162.902 90.642) (end 159.26 87) (width 0.2) (layer "F.Cu") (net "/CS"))
 (segment (start 197.558 90.642) (end 162.902 90.642) (width 0.2) (layer "F.Cu") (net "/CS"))
 (segment (start 198.62 89.58) (end 197.558 90.642) (width 0.2) (layer "F.Cu") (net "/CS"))
 (segment (start 198.180105 77.942) (end 200.710214 77.942) (width 0.2) (layer "B.Cu") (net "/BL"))
 (segment (start 200.971 76.078786) (end 200.710214 75.818) (width 0.2) (layer "B.Cu") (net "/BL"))
 (segment (start 167.902 75.818) (end 156.72 87) (width 0.2) (layer "B.Cu") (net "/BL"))
 (segment (start 197.142 78.980105) (end 198.180105 77.942) (width 0.2) (layer "B.Cu") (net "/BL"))
 (segment (start 198.62 92.12) (end 197.142 90.642) (width 0.2) (layer "B.Cu") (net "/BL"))
 (segment (start 200.710214 75.818) (end 167.902 75.818) (width 0.2) (layer "B.Cu") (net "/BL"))
 (segment (start 200.971 77.681214) (end 200.971 76.078786) (width 0.2) (layer "B.Cu") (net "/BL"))
 (segment (start 200.710214 77.942) (end 200.971 77.681214) (width 0.2) (layer "B.Cu") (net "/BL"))
 (segment (start 197.142 90.642) (end 197.142 78.980105) (width 0.2) (layer "B.Cu") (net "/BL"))
 (segment (start 183.38 89.58) (end 162.753654 89.58) (width 0.2) (layer "F.Cu") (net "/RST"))
 (segment (start 161.323654 85.85) (end 163.19 85.85) (width 0.2) (layer "F.Cu") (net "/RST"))
 (segment (start 160.65 86.523654) (end 161.323654 85.85) (width 0.2) (layer "F.Cu") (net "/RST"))
 (segment (start 163.19 85.85) (end 164.34 87) (width 0.2) (layer "F.Cu") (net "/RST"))
 (segment (start 160.65 87.476346) (end 160.65 86.523654) (width 0.2) (layer "F.Cu") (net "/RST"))
 (segment (start 162.753654 89.58) (end 160.65 87.476346) (width 0.2) (layer "F.Cu") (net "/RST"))
 (segment (start 180.24 83.9) (end 183.38 87.04) (width 0.2) (layer "F.Cu") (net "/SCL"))
 (segment (start 173.42 83) (end 177 83) (width 0.2) (layer "F.Cu") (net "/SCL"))
 (segment (start 179 83.9) (end 180.24 83.9) (width 0.2) (layer "F.Cu") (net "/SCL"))
 (segment (start 169.42 87) (end 173.42 83) (width 0.2) (layer "F.Cu") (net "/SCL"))
 (via (at 179 83.9) (size 0.6) (drill 0.3) (layers "F.Cu" "B.Cu") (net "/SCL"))
 (via (at 177 83) (size 0.6) (drill 0.3) (layers "F.Cu" "B.Cu") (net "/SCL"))
 (segment (start 177 83) (end 177.9 83.9) (width 0.2) (layer "B.Cu") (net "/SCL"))
 (segment (start 177.9 83.9) (end 179 83.9) (width 0.2) (layer "B.Cu") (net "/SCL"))
 (segment (start 169.38 84.5) (end 166.88 87) (width 0.2) (layer "B.Cu") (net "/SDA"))
 (segment (start 183.38 84.5) (end 169.38 84.5) (width 0.2) (layer "B.Cu") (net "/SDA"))
 (segment (start 173.11 85.85) (end 171.96 87) (width 0.2) (layer "B.Cu") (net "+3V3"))
 (segment (start 183.38 81.96) (end 184.442 83.022) (width 0.2) (layer "B.Cu") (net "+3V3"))
 (segment (start 184.442 84.939895) (end 183.531895 85.85) (width 0.2) (layer "B.Cu") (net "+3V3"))
 (segment (start 184.442 83.022) (end 184.442 84.939895) (width 0.2) (layer "B.Cu") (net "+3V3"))
 (segment (start 183.531895 85.85) (end 173.11 85.85) (width 0.2) (layer "B.Cu") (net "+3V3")))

